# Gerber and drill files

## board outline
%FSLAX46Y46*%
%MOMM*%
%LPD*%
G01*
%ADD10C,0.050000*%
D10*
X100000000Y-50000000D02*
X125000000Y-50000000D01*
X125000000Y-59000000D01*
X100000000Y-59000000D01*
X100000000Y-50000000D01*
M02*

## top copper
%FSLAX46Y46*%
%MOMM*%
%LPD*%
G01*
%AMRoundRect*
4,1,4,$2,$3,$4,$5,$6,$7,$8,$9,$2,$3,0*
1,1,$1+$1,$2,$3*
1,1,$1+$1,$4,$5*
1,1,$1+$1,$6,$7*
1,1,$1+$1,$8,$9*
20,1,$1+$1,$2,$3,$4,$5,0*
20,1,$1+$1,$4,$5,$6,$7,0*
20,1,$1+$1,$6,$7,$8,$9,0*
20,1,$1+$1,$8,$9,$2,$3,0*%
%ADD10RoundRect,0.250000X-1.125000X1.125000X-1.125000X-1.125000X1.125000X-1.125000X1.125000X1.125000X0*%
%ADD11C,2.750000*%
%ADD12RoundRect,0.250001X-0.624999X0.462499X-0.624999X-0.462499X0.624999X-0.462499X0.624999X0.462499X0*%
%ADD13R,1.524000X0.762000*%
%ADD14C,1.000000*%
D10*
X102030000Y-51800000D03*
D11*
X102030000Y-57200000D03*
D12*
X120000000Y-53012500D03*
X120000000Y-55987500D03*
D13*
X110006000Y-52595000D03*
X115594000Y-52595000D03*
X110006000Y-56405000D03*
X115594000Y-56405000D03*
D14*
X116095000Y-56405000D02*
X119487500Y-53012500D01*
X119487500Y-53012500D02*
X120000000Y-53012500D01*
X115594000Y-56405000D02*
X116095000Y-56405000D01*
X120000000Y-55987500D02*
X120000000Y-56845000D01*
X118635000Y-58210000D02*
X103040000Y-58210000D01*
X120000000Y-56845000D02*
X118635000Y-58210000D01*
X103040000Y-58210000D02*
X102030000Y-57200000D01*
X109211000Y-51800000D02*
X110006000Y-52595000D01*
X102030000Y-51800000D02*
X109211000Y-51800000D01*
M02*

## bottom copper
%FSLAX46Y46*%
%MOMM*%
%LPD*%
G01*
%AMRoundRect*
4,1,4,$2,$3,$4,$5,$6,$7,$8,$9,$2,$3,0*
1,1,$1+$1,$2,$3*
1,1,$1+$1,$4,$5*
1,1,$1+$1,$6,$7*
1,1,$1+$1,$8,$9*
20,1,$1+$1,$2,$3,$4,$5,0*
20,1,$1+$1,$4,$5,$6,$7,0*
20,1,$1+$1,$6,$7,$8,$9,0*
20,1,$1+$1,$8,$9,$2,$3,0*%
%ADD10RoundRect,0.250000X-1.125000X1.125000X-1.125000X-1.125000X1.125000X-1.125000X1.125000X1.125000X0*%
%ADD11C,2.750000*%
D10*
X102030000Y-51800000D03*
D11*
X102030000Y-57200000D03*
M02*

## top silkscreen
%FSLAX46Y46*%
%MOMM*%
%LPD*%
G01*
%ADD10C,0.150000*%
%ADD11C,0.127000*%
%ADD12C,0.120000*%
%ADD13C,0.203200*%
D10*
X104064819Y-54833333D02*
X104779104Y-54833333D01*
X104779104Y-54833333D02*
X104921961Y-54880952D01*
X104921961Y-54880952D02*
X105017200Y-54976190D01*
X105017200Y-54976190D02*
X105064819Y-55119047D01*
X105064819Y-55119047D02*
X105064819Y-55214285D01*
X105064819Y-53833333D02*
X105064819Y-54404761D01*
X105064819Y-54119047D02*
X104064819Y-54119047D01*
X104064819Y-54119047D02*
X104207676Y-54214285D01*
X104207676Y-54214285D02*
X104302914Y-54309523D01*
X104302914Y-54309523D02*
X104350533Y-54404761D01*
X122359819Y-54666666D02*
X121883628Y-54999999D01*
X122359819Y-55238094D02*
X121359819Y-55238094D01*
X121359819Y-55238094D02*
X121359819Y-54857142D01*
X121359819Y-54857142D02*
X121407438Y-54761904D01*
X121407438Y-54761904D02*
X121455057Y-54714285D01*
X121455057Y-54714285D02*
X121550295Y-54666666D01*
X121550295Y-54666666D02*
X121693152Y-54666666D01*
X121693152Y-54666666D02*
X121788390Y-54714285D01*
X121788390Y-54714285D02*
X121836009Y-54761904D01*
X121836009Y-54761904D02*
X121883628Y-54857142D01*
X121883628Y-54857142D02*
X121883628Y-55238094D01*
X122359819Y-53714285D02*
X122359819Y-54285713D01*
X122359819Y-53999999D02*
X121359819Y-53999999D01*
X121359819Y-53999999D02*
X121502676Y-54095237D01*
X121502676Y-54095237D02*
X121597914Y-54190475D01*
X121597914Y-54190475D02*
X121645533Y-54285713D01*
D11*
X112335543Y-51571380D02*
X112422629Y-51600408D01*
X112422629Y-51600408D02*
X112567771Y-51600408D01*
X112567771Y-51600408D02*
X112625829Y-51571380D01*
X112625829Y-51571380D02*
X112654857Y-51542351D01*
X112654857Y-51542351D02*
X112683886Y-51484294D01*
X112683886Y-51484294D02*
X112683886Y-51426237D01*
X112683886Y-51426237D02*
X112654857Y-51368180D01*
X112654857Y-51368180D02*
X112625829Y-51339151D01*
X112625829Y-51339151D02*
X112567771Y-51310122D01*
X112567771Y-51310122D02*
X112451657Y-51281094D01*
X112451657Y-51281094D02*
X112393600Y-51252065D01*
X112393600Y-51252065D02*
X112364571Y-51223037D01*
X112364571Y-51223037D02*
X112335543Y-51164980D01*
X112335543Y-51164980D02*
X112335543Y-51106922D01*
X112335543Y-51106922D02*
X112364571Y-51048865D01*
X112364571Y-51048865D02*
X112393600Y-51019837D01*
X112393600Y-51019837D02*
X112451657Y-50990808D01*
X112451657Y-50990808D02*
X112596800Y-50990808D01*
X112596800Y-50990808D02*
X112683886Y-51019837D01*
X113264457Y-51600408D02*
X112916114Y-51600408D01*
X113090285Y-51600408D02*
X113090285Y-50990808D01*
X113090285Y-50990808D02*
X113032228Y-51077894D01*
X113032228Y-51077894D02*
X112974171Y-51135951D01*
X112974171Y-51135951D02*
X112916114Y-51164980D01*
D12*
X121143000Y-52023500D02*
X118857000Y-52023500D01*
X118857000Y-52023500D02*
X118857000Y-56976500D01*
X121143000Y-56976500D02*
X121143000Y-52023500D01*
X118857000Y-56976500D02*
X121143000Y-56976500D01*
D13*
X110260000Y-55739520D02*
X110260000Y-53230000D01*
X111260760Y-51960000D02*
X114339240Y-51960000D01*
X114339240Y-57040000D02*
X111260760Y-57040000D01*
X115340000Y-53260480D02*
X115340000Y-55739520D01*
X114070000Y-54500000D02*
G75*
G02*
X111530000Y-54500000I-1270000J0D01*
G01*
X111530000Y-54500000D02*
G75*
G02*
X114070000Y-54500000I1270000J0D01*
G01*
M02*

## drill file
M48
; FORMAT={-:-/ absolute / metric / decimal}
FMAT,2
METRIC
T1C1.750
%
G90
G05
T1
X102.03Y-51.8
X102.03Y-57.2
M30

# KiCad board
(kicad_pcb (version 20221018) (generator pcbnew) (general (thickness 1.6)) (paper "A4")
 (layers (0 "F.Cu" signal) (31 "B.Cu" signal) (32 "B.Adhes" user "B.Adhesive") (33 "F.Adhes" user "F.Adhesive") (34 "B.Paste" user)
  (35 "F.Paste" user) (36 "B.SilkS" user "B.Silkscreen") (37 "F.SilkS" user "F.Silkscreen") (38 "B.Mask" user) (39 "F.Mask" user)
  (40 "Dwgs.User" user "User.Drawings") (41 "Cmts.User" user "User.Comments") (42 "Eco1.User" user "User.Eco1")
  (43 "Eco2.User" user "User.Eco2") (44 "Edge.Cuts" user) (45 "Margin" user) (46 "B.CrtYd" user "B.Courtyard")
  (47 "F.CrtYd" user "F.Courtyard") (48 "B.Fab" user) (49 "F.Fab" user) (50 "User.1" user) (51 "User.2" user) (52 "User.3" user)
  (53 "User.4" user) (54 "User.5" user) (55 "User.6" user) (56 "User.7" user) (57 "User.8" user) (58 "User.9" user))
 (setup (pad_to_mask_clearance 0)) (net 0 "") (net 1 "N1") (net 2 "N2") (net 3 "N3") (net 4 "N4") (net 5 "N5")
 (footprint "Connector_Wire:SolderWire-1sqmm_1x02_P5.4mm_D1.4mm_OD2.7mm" (layer "F.Cu") (at 102.03 51.8 -90)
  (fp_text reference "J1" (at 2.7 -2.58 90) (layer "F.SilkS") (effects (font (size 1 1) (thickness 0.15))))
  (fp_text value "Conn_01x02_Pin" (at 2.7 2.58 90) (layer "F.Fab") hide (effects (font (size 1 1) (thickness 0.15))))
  (pad "1" thru_hole roundrect (at 0 0 270) (size 2.75 2.75) (drill 1.75) (layers "*.Cu" "*.Mask") (roundrect_rratio 0.09090909091)
   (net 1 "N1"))
  (pad "2" thru_hole circle (at 5.4 0 270) (size 2.75 2.75) (drill 1.75) (layers "*.Cu" "*.Mask") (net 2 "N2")))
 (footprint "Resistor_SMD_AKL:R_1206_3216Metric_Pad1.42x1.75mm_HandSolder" (layer "F.Cu") (at 120 54.5 -90)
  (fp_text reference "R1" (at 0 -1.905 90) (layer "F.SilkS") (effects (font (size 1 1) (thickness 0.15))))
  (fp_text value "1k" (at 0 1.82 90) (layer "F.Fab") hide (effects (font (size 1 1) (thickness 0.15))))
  (fp_line (start -2.4765 -1.143) (end -2.4765 1.143) (stroke (width 0.12) (type solid)) (layer "F.SilkS"))
  (fp_line (start -2.4765 1.143) (end 2.4765 1.143) (stroke (width 0.12) (type solid)) (layer "F.SilkS"))
  (fp_line (start 2.4765 -1.143) (end -2.4765 -1.143) (stroke (width 0.12) (type solid)) (layer "F.SilkS"))
  (fp_line (start 2.4765 1.143) (end 2.4765 -1.143) (stroke (width 0.12) (type solid)) (layer "F.SilkS"))
  (pad "1" smd roundrect (at -1.4875 0 270) (size 1.425 1.75) (layers "F.Cu" "F.Paste" "F.Mask") (roundrect_rratio 0.1754392982)
   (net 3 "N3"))
  (pad "2" smd roundrect (at 1.4875 0 270) (size 1.425 1.75) (layers "F.Cu" "F.Paste" "F.Mask") (roundrect_rratio 0.1754392982) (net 2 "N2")))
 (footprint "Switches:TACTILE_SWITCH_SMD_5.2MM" (layer "F.Cu") (at 112.8 54.5)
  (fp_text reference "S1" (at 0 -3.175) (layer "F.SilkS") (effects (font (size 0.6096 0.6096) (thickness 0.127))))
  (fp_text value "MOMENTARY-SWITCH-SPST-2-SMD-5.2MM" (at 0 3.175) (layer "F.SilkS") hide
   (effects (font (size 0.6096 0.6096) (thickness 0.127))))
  (fp_line (start -2.54 1.23952) (end -2.54 -1.27) (stroke (width 0.2032) (type solid)) (layer "F.SilkS"))
  (fp_line (start -1.53924 -2.54) (end 1.53924 -2.54) (stroke (width 0.2032) (type solid)) (layer "F.SilkS"))
  (fp_line (start 1.53924 2.54) (end -1.53924 2.54) (stroke (width 0.2032) (type solid)) (layer "F.SilkS"))
  (fp_line (start 2.54 -1.23952) (end 2.54 1.23952) (stroke (width 0.2032) (type solid)) (layer "F.SilkS"))
  (fp_circle (center 0 0) (end 0 -1.27) (stroke (width 0.2032) (type solid)) (fill none) (layer "F.SilkS"))
  (pad "1" smd rect (at -2.794 -1.905 90) (size 0.762 1.524) (layers "F.Cu" "F.Paste" "F.Mask") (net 1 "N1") (solder_mask_margin 0.1016))
  (pad "2" smd rect (at 2.794 -1.905 90) (size 0.762 1.524) (layers "F.Cu" "F.Paste" "F.Mask") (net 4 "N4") (solder_mask_margin 0.1016))
  (pad "3" smd rect (at -2.794 1.905 90) (size 0.762 1.524) (layers "F.Cu" "F.Paste" "F.Mask") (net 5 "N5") (solder_mask_margin 0.1016))
  (pad "4" smd rect (at 2.794 1.905 90) (size 0.762 1.524) (layers "F.Cu" "F.Paste" "F.Mask") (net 3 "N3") (solder_mask_margin 0.1016)))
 (gr_rect locked (start 100 50) (end 125 59) (stroke (width 0.05) (type default)) (fill none) (layer "Edge.Cuts"))
 (segment (start 116.095 56.405) (end 119.4875 53.0125) (width 1) (layer "F.Cu") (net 3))
 (segment (start 119.4875 53.0125) (end 120 53.0125) (width 1) (layer "F.Cu") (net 3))
 (segment (start 115.594 56.405) (end 116.095 56.405) (width 1) (layer "F.Cu") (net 3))
 (segment (start 120 55.9875) (end 120 56.845) (width 1) (layer "F.Cu") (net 2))
 (segment (start 118.635 58.21) (end 103.04 58.21) (width 1) (layer "F.Cu") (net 2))
 (segment (start 120 56.845) (end 118.635 58.21) (width 1) (layer "F.Cu") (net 2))
 (segment (start 103.04 58.21) (end 102.03 57.2) (width 1) (layer "F.Cu") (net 2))
 (segment (start 109.211 51.8) (end 110.006 52.595) (width 1) (layer "F.Cu") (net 1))
 (segment (start 102.03 51.8) (end 109.211 51.8) (width 1) (layer "F.Cu") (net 1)))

